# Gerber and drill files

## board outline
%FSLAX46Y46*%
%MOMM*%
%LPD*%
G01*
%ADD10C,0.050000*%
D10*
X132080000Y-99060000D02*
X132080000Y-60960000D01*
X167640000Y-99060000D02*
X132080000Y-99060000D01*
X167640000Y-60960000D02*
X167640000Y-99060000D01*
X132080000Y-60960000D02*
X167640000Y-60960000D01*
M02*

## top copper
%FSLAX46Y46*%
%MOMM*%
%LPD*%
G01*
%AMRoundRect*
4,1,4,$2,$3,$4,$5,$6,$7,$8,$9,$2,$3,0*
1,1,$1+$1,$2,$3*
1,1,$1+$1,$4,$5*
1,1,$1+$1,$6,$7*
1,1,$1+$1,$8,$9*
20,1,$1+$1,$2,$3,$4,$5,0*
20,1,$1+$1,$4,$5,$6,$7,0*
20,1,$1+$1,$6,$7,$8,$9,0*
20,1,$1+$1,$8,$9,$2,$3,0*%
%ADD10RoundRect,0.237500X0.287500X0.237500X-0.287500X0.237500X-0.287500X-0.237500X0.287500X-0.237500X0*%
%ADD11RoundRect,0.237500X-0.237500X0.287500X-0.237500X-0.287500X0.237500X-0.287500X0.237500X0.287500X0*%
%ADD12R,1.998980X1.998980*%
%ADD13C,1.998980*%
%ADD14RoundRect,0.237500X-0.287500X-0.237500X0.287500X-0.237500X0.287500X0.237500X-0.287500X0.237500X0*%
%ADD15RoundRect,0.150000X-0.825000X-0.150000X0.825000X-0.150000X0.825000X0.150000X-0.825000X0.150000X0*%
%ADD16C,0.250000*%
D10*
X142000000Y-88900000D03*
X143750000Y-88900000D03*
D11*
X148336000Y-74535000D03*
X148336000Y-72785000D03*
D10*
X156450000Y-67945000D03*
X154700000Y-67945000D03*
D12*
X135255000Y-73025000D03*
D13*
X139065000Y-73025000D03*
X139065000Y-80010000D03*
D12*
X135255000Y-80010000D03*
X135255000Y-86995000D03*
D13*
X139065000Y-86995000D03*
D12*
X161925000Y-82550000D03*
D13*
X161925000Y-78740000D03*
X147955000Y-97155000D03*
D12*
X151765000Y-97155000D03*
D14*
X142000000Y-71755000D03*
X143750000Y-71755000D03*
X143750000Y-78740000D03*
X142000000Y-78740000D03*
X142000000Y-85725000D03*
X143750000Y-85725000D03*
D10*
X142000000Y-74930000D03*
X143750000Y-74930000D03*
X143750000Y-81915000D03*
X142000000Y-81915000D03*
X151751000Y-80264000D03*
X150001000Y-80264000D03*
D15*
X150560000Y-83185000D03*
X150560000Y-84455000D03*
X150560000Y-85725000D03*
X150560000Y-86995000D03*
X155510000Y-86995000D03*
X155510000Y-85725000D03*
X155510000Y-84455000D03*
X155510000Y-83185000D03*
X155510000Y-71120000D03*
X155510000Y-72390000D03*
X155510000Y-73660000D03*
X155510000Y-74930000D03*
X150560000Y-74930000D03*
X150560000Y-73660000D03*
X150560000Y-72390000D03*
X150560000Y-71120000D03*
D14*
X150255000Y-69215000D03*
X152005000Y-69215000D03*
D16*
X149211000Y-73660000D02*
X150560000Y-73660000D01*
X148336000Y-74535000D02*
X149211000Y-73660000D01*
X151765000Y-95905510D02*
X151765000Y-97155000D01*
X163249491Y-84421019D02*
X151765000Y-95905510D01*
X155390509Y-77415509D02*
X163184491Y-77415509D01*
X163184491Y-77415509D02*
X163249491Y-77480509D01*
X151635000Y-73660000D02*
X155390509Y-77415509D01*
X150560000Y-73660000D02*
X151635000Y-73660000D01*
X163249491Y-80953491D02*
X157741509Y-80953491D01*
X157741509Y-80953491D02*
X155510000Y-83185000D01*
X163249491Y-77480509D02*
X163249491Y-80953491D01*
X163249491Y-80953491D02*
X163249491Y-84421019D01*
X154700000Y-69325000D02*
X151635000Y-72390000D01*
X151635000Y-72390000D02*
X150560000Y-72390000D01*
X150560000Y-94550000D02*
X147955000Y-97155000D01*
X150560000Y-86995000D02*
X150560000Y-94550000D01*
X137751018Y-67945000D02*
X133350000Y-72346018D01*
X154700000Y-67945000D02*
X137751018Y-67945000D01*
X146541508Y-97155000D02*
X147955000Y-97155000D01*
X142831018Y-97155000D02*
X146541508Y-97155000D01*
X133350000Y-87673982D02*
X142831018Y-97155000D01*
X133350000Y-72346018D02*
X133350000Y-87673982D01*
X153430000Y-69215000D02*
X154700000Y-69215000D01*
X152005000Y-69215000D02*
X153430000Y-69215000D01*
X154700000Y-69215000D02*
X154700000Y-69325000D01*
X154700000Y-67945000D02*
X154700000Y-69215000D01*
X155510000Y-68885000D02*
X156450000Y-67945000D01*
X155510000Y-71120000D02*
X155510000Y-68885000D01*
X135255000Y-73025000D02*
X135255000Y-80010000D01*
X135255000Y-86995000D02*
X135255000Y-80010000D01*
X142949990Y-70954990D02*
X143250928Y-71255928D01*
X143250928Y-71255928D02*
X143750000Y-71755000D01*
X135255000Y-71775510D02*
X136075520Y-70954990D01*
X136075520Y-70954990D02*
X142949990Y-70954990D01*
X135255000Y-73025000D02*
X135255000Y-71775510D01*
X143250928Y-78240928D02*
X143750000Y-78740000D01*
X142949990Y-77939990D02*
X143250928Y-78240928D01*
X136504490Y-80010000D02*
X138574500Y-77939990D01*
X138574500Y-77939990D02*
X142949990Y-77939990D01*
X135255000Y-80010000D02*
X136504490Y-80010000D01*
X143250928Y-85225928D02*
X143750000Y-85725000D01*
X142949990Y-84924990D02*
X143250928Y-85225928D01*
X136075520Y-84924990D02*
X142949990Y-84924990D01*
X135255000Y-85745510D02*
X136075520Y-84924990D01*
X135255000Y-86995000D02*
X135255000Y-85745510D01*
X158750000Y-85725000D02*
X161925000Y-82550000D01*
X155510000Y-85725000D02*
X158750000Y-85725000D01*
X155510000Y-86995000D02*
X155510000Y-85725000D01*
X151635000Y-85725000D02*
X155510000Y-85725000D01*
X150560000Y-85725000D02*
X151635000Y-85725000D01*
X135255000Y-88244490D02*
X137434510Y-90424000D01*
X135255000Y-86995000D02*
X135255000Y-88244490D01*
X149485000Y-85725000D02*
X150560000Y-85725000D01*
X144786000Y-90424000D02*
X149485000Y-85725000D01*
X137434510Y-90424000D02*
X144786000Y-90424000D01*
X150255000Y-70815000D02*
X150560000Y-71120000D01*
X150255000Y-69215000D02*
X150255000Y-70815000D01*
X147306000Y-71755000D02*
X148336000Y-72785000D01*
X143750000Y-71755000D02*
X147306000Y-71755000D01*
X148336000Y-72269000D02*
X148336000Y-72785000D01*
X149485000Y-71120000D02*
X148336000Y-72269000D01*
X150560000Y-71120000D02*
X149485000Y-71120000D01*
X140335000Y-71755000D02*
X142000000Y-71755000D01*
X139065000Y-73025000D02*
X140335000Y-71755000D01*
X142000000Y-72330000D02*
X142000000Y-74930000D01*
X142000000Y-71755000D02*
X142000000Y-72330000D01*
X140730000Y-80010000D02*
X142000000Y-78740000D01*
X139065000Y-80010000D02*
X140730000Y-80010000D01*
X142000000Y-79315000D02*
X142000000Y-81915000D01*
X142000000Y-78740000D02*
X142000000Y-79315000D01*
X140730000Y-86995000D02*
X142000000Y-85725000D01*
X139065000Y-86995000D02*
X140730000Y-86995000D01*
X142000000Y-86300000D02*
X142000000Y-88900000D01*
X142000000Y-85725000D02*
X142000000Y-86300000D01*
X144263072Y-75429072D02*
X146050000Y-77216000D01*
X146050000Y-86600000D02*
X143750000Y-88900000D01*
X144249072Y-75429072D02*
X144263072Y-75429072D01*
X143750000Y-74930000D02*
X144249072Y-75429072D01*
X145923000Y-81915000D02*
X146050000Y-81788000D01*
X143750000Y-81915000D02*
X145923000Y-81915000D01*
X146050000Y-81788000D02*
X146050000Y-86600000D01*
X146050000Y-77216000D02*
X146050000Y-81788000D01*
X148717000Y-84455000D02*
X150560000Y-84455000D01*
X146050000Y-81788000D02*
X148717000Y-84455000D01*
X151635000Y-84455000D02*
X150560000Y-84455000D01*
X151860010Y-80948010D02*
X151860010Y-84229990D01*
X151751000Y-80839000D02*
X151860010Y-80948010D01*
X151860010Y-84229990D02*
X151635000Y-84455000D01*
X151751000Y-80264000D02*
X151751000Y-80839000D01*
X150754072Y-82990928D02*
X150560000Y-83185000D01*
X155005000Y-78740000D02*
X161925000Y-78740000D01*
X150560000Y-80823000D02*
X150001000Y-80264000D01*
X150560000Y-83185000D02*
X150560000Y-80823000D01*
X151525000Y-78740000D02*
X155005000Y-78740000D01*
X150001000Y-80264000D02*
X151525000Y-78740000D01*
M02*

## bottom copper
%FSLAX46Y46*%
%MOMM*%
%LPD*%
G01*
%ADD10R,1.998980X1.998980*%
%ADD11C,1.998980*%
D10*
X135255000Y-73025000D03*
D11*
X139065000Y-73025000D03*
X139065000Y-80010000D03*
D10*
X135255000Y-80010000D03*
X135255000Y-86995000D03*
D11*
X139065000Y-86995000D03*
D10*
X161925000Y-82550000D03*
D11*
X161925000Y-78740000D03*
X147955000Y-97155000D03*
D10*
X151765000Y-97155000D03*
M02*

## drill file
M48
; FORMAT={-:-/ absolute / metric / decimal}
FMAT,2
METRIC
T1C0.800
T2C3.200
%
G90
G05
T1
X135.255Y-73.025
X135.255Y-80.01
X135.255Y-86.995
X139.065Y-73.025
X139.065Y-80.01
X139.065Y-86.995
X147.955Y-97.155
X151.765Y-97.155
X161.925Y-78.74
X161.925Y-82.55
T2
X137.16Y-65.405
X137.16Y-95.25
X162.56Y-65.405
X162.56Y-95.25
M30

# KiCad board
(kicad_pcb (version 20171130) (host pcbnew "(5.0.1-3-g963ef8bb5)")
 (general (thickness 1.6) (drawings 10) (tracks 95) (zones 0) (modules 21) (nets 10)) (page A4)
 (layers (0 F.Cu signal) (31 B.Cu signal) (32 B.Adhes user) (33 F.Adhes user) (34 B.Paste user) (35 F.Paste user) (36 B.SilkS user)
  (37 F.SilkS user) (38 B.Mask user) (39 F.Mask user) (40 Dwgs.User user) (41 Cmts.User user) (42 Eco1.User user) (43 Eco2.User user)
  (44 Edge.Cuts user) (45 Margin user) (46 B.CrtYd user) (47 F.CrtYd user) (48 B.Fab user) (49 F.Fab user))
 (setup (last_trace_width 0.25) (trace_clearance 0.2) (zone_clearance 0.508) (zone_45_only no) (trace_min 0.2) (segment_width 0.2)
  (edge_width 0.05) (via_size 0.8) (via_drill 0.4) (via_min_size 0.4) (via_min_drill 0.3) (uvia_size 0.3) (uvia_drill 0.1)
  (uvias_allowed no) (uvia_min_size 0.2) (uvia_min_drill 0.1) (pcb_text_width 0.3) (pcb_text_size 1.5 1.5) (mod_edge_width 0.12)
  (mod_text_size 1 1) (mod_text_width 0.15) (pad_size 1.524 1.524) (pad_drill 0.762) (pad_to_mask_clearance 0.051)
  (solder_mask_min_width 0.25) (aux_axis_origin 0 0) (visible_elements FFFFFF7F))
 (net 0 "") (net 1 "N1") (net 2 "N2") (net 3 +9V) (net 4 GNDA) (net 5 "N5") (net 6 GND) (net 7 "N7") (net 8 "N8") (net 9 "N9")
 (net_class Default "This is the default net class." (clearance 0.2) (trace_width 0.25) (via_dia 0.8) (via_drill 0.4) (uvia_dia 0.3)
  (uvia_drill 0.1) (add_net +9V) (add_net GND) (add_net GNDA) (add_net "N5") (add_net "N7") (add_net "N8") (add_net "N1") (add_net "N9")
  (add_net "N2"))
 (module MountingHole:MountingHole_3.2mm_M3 (layer F.Cu) (at 162.56 95.25)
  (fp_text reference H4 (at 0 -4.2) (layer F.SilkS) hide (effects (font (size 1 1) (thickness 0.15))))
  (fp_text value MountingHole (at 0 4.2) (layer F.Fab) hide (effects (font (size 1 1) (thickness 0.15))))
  (pad 1 np_thru_hole circle (at 0 0) (size 3.2 3.2) (drill 3.2) (layers *.Cu *.Mask)))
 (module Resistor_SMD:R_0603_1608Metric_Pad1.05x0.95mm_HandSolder (layer F.Cu) (at 142.875 88.9 180)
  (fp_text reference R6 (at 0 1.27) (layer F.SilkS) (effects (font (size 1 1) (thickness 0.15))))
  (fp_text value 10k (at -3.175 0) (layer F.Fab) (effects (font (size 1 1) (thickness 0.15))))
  (pad 2 smd roundrect (at 0.875 0 180) (size 1.05 0.95) (layers F.Cu F.Paste F.Mask) (roundrect_rratio 0.25) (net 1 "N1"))
  (pad 1 smd roundrect (at -0.875 0 180) (size 1.05 0.95) (layers F.Cu F.Paste F.Mask) (roundrect_rratio 0.25) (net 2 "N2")))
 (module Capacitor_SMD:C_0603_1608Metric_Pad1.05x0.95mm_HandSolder (layer F.Cu) (at 148.336 73.66 270)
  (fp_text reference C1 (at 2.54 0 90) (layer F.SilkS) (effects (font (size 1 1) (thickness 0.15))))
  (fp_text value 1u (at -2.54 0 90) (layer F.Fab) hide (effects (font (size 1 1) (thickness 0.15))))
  (pad 2 smd roundrect (at 0.875 0 270) (size 1.05 0.95) (layers F.Cu F.Paste F.Mask) (roundrect_rratio 0.25) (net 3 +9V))
  (pad 1 smd roundrect (at -0.875 0 270) (size 1.05 0.95) (layers F.Cu F.Paste F.Mask) (roundrect_rratio 0.25) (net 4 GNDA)))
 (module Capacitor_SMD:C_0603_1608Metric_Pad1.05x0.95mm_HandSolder (layer F.Cu) (at 155.575 67.945 180)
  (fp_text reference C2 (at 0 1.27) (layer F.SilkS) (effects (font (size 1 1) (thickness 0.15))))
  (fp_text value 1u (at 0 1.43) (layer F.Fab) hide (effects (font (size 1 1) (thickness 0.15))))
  (pad 1 smd roundrect (at -0.875 0 180) (size 1.05 0.95) (layers F.Cu F.Paste F.Mask) (roundrect_rratio 0.25) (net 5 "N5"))
  (pad 2 smd roundrect (at 0.875 0 180) (size 1.05 0.95) (layers F.Cu F.Paste F.Mask) (roundrect_rratio 0.25) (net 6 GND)))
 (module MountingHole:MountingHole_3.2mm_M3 (layer F.Cu) (at 137.16 65.405)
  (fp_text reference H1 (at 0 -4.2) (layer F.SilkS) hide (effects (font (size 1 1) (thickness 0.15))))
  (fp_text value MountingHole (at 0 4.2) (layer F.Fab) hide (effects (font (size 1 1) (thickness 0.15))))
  (pad 1 np_thru_hole circle (at 0 0) (size 3.2 3.2) (drill 3.2) (layers *.Cu *.Mask)))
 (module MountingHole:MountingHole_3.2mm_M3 (layer F.Cu) (at 162.56 65.405)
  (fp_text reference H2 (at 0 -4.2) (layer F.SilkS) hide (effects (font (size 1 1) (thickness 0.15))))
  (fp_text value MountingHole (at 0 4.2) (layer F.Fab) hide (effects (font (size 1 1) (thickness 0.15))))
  (pad 1 np_thru_hole circle (at 0 0) (size 3.2 3.2) (drill 3.2) (layers *.Cu *.Mask)))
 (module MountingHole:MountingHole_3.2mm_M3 (layer F.Cu) (at 137.16 95.25)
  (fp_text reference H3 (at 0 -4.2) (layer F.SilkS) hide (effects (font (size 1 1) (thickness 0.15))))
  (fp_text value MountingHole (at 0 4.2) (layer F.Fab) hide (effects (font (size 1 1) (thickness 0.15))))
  (pad 1 np_thru_hole circle (at 0 0) (size 3.2 3.2) (drill 3.2) (layers *.Cu *.Mask)))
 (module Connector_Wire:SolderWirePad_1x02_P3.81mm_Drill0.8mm (layer F.Cu) (at 135.255 73.025)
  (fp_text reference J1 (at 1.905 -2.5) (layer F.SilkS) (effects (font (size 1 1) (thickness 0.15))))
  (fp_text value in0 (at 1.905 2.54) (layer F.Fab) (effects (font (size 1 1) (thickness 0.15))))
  (pad 1 thru_hole rect (at 0 0) (size 1.99898 1.99898) (drill 0.8001) (layers *.Cu *.Mask) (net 4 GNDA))
  (pad 2 thru_hole circle (at 3.81 0) (size 1.99898 1.99898) (drill 0.8001) (layers *.Cu *.Mask) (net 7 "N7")))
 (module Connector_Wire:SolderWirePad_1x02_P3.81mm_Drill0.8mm (layer F.Cu) (at 135.255 80.01)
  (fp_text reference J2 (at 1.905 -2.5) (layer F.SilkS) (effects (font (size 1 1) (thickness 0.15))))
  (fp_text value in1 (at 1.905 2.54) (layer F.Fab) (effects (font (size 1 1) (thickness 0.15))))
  (pad 2 thru_hole circle (at 3.81 0) (size 1.99898 1.99898) (drill 0.8001) (layers *.Cu *.Mask) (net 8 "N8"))
  (pad 1 thru_hole rect (at 0 0) (size 1.99898 1.99898) (drill 0.8001) (layers *.Cu *.Mask) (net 4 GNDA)))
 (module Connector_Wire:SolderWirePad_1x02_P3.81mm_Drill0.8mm (layer F.Cu) (at 135.255 86.995)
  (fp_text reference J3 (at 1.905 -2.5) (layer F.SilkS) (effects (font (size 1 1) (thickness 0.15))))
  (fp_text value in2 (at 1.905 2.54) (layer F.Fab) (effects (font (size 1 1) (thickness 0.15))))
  (pad 1 thru_hole rect (at 0 0) (size 1.99898 1.99898) (drill 0.8001) (layers *.Cu *.Mask) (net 4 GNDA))
  (pad 2 thru_hole circle (at 3.81 0) (size 1.99898 1.99898) (drill 0.8001) (layers *.Cu *.Mask) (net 1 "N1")))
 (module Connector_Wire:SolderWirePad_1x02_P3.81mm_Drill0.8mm (layer F.Cu) (at 161.925 82.55 90)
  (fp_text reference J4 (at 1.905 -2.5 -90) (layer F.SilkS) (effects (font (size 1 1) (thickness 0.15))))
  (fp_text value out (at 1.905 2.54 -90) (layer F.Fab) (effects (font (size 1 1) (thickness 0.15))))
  (pad 1 thru_hole rect (at 0 0 90) (size 1.99898 1.99898) (drill 0.8001) (layers *.Cu *.Mask) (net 4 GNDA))
  (pad 2 thru_hole circle (at 3.81 0 90) (size 1.99898 1.99898) (drill 0.8001) (layers *.Cu *.Mask) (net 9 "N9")))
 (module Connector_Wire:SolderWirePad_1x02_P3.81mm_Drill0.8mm (layer F.Cu) (at 151.765 97.155 180)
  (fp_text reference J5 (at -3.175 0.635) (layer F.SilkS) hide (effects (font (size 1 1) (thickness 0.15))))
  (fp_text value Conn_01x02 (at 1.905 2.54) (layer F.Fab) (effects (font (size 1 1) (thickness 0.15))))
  (pad 2 thru_hole circle (at 3.81 0 180) (size 1.99898 1.99898) (drill 0.8001) (layers *.Cu *.Mask) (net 6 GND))
  (pad 1 thru_hole rect (at 0 0 180) (size 1.99898 1.99898) (drill 0.8001) (layers *.Cu *.Mask) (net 3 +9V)))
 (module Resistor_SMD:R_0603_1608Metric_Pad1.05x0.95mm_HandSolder (layer F.Cu) (at 142.875 71.755)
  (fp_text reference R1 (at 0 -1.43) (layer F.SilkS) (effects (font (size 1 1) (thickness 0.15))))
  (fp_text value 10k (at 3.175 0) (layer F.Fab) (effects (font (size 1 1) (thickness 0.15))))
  (pad 1 smd roundrect (at -0.875 0) (size 1.05 0.95) (layers F.Cu F.Paste F.Mask) (roundrect_rratio 0.25) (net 7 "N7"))
  (pad 2 smd roundrect (at 0.875 0) (size 1.05 0.95) (layers F.Cu F.Paste F.Mask) (roundrect_rratio 0.25) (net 4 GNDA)))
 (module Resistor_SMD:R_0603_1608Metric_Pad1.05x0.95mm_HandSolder (layer F.Cu) (at 142.875 78.74)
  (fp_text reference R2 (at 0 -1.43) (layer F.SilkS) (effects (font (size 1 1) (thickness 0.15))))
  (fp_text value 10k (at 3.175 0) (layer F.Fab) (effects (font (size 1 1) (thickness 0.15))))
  (pad 2 smd roundrect (at 0.875 0) (size 1.05 0.95) (layers F.Cu F.Paste F.Mask) (roundrect_rratio 0.25) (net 4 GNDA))
  (pad 1 smd roundrect (at -0.875 0) (size 1.05 0.95) (layers F.Cu F.Paste F.Mask) (roundrect_rratio 0.25) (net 8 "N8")))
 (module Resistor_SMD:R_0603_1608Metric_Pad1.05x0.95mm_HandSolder (layer F.Cu) (at 142.875 85.725)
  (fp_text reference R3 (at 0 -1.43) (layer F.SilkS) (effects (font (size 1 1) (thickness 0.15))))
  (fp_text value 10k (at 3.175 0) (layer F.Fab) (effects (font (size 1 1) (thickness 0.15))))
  (pad 1 smd roundrect (at -0.875 0) (size 1.05 0.95) (layers F.Cu F.Paste F.Mask) (roundrect_rratio 0.25) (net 1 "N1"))
  (pad 2 smd roundrect (at 0.875 0) (size 1.05 0.95) (layers F.Cu F.Paste F.Mask) (roundrect_rratio 0.25) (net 4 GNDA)))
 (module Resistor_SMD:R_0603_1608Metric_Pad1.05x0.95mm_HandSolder (layer F.Cu) (at 142.875 74.93 180)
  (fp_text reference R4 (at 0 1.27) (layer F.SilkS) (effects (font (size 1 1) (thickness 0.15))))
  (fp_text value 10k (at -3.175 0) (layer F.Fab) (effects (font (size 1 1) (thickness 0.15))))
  (pad 2 smd roundrect (at 0.875 0 180) (size 1.05 0.95) (layers F.Cu F.Paste F.Mask) (roundrect_rratio 0.25) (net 7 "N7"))
  (pad 1 smd roundrect (at -0.875 0 180) (size 1.05 0.95) (layers F.Cu F.Paste F.Mask) (roundrect_rratio 0.25) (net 2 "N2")))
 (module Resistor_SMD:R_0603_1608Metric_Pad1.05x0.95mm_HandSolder (layer F.Cu) (at 142.875 81.915 180)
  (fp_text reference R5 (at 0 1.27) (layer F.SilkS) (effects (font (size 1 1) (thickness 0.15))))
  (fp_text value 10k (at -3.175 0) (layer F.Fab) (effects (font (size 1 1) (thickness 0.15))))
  (pad 1 smd roundrect (at -0.875 0 180) (size 1.05 0.95) (layers F.Cu F.Paste F.Mask) (roundrect_rratio 0.25) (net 2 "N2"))
  (pad 2 smd roundrect (at 0.875 0 180) (size 1.05 0.95) (layers F.Cu F.Paste F.Mask) (roundrect_rratio 0.25) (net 8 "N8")))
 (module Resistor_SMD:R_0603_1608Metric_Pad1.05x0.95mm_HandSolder (layer F.Cu) (at 150.876 80.264 180)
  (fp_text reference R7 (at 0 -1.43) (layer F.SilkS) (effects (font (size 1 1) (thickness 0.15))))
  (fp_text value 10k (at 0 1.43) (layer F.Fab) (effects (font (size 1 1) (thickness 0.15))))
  (pad 1 smd roundrect (at -0.875 0 180) (size 1.05 0.95) (layers F.Cu F.Paste F.Mask) (roundrect_rratio 0.25) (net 2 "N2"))
  (pad 2 smd roundrect (at 0.875 0 180) (size 1.05 0.95) (layers F.Cu F.Paste F.Mask) (roundrect_rratio 0.25) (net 9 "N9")))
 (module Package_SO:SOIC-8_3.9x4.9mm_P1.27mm (layer F.Cu) (at 153.035 85.09)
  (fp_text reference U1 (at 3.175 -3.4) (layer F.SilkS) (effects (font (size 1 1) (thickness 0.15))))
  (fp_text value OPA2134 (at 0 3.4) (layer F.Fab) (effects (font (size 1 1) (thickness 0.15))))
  (pad 1 smd roundrect (at -2.475 -1.905) (size 1.95 0.6) (layers F.Cu F.Paste F.Mask) (roundrect_rratio 0.25) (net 9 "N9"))
  (pad 2 smd roundrect (at -2.475 -0.635) (size 1.95 0.6) (layers F.Cu F.Paste F.Mask) (roundrect_rratio 0.25) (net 2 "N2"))
  (pad 3 smd roundrect (at -2.475 0.635) (size 1.95 0.6) (layers F.Cu F.Paste F.Mask) (roundrect_rratio 0.25) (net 4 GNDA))
  (pad 4 smd roundrect (at -2.475 1.905) (size 1.95 0.6) (layers F.Cu F.Paste F.Mask) (roundrect_rratio 0.25) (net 6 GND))
  (pad 5 smd roundrect (at 2.475 1.905) (size 1.95 0.6) (layers F.Cu F.Paste F.Mask) (roundrect_rratio 0.25) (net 4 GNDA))
  (pad 6 smd roundrect (at 2.475 0.635) (size 1.95 0.6) (layers F.Cu F.Paste F.Mask) (roundrect_rratio 0.25) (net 4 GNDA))
  (pad 7 smd roundrect (at 2.475 -0.635) (size 1.95 0.6) (layers F.Cu F.Paste F.Mask) (roundrect_rratio 0.25))
  (pad 8 smd roundrect (at 2.475 -1.905) (size 1.95 0.6) (layers F.Cu F.Paste F.Mask) (roundrect_rratio 0.25) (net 3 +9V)))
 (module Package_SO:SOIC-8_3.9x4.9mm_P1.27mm (layer F.Cu) (at 153.035 73.025)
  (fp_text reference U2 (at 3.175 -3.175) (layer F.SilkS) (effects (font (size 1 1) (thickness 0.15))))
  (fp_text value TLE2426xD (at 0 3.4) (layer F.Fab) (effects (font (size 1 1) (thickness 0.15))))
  (pad 8 smd roundrect (at 2.475 -1.905) (size 1.95 0.6) (layers F.Cu F.Paste F.Mask) (roundrect_rratio 0.25) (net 5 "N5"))
  (pad 7 smd roundrect (at 2.475 -0.635) (size 1.95 0.6) (layers F.Cu F.Paste F.Mask) (roundrect_rratio 0.25))
  (pad 6 smd roundrect (at 2.475 0.635) (size 1.95 0.6) (layers F.Cu F.Paste F.Mask) (roundrect_rratio 0.25))
  (pad 5 smd roundrect (at 2.475 1.905) (size 1.95 0.6) (layers F.Cu F.Paste F.Mask) (roundrect_rratio 0.25))
  (pad 4 smd roundrect (at -2.475 1.905) (size 1.95 0.6) (layers F.Cu F.Paste F.Mask) (roundrect_rratio 0.25))
  (pad 3 smd roundrect (at -2.475 0.635) (size 1.95 0.6) (layers F.Cu F.Paste F.Mask) (roundrect_rratio 0.25) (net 3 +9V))
  (pad 2 smd roundrect (at -2.475 -0.635) (size 1.95 0.6) (layers F.Cu F.Paste F.Mask) (roundrect_rratio 0.25) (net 6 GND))
  (pad 1 smd roundrect (at -2.475 -1.905) (size 1.95 0.6) (layers F.Cu F.Paste F.Mask) (roundrect_rratio 0.25) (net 4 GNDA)))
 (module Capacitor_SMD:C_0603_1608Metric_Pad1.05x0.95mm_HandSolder (layer F.Cu) (at 151.13 69.215)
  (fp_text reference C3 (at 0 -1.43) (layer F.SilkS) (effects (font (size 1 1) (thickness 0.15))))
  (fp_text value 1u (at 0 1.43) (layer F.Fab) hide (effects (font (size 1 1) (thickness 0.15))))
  (pad 1 smd roundrect (at -0.875 0) (size 1.05 0.95) (layers F.Cu F.Paste F.Mask) (roundrect_rratio 0.25) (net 4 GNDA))
  (pad 2 smd roundrect (at 0.875 0) (size 1.05 0.95) (layers F.Cu F.Paste F.Mask) (roundrect_rratio 0.25) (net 6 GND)))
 (gr_line (start 132.08 99.06) (end 132.08 60.96) (layer Edge.Cuts) (width 0.05))
 (gr_line (start 167.64 99.06) (end 132.08 99.06) (layer Edge.Cuts) (width 0.05))
 (gr_line (start 167.64 60.96) (end 167.64 99.06) (layer Edge.Cuts) (width 0.05))
 (gr_line (start 132.08 60.96) (end 167.64 60.96) (layer Edge.Cuts) (width 0.05))
 (segment (start 149.211 73.66) (end 150.56 73.66) (width 0.25) (layer F.Cu) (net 3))
 (segment (start 148.336 74.535) (end 149.211 73.66) (width 0.25) (layer F.Cu) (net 3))
 (segment (start 151.765 95.90551) (end 151.765 97.155) (width 0.25) (layer F.Cu) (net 3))
 (segment (start 163.249491 84.421019) (end 151.765 95.90551) (width 0.25) (layer F.Cu) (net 3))
 (segment (start 155.390509 77.415509) (end 163.184491 77.415509) (width 0.25) (layer F.Cu) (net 3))
 (segment (start 163.184491 77.415509) (end 163.249491 77.480509) (width 0.25) (layer F.Cu) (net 3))
 (segment (start 151.635 73.66) (end 155.390509 77.415509) (width 0.25) (layer F.Cu) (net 3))
 (segment (start 150.56 73.66) (end 151.635 73.66) (width 0.25) (layer F.Cu) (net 3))
 (segment (start 163.249491 80.953491) (end 157.741509 80.953491) (width 0.25) (layer F.Cu) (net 3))
 (segment (start 157.741509 80.953491) (end 155.51 83.185) (width 0.25) (layer F.Cu) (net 3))
 (segment (start 163.249491 77.480509) (end 163.249491 80.953491) (width 0.25) (layer F.Cu) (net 3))
 (segment (start 163.249491 80.953491) (end 163.249491 84.421019) (width 0.25) (layer F.Cu) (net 3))
 (segment (start 154.7 69.325) (end 151.635 72.39) (width 0.25) (layer F.Cu) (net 6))
 (segment (start 151.635 72.39) (end 150.56 72.39) (width 0.25) (layer F.Cu) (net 6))
 (segment (start 150.56 94.55) (end 147.955 97.155) (width 0.25) (layer F.Cu) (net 6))
 (segment (start 150.56 86.995) (end 150.56 94.55) (width 0.25) (layer F.Cu) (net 6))
 (segment (start 137.751018 67.945) (end 133.35 72.346018) (width 0.25) (layer F.Cu) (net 6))
 (segment (start 154.7 67.945) (end 137.751018 67.945) (width 0.25) (layer F.Cu) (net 6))
 (segment (start 146.541508 97.155) (end 147.955 97.155) (width 0.25) (layer F.Cu) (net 6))
 (segment (start 142.831018 97.155) (end 146.541508 97.155) (width 0.25) (layer F.Cu) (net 6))
 (segment (start 133.35 87.673982) (end 142.831018 97.155) (width 0.25) (layer F.Cu) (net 6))
 (segment (start 133.35 72.346018) (end 133.35 87.673982) (width 0.25) (layer F.Cu) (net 6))
 (segment (start 153.43 69.215) (end 154.7 69.215) (width 0.25) (layer F.Cu) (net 6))
 (segment (start 152.005 69.215) (end 153.43 69.215) (width 0.25) (layer F.Cu) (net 6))
 (segment (start 154.7 69.215) (end 154.7 69.325) (width 0.25) (layer F.Cu) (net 6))
 (segment (start 154.7 67.945) (end 154.7 69.215) (width 0.25) (layer F.Cu) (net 6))
 (segment (start 155.51 68.885) (end 156.45 67.945) (width 0.25) (layer F.Cu) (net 5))
 (segment (start 155.51 71.12) (end 155.51 68.885) (width 0.25) (layer F.Cu) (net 5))
 (segment (start 135.255 73.025) (end 135.255 80.01) (width 0.25) (layer F.Cu) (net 4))
 (segment (start 135.255 86.995) (end 135.255 80.01) (width 0.25) (layer F.Cu) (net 4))
 (segment (start 142.94999 70.95499) (end 143.250928 71.255928) (width 0.25) (layer F.Cu) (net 4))
 (segment (start 143.250928 71.255928) (end 143.75 71.755) (width 0.25) (layer F.Cu) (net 4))
 (segment (start 135.255 71.77551) (end 136.07552 70.95499) (width 0.25) (layer F.Cu) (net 4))
 (segment (start 136.07552 70.95499) (end 142.94999 70.95499) (width 0.25) (layer F.Cu) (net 4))
 (segment (start 135.255 73.025) (end 135.255 71.77551) (width 0.25) (layer F.Cu) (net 4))
 (segment (start 143.250928 78.240928) (end 143.75 78.74) (width 0.25) (layer F.Cu) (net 4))
 (segment (start 142.94999 77.93999) (end 143.250928 78.240928) (width 0.25) (layer F.Cu) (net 4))
 (segment (start 136.50449 80.01) (end 138.5745 77.93999) (width 0.25) (layer F.Cu) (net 4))
 (segment (start 138.5745 77.93999) (end 142.94999 77.93999) (width 0.25) (layer F.Cu) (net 4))
 (segment (start 135.255 80.01) (end 136.50449 80.01) (width 0.25) (layer F.Cu) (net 4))
 (segment (start 143.250928 85.225928) (end 143.75 85.725) (width 0.25) (layer F.Cu) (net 4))
 (segment (start 142.94999 84.92499) (end 143.250928 85.225928) (width 0.25) (layer F.Cu) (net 4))
 (segment (start 136.07552 84.92499) (end 142.94999 84.92499) (width 0.25) (layer F.Cu) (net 4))
 (segment (start 135.255 85.74551) (end 136.07552 84.92499) (width 0.25) (layer F.Cu) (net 4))
 (segment (start 135.255 86.995) (end 135.255 85.74551) (width 0.25) (layer F.Cu) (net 4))
 (segment (start 158.75 85.725) (end 161.925 82.55) (width 0.25) (layer F.Cu) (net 4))
 (segment (start 155.51 85.725) (end 158.75 85.725) (width 0.25) (layer F.Cu) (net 4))
 (segment (start 155.51 86.995) (end 155.51 85.725) (width 0.25) (layer F.Cu) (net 4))
 (segment (start 151.635 85.725) (end 155.51 85.725) (width 0.25) (layer F.Cu) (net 4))
 (segment (start 150.56 85.725) (end 151.635 85.725) (width 0.25) (layer F.Cu) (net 4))
 (segment (start 135.255 88.24449) (end 137.43451 90.424) (width 0.25) (layer F.Cu) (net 4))
 (segment (start 135.255 86.995) (end 135.255 88.24449) (width 0.25) (layer F.Cu) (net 4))
 (segment (start 149.485 85.725) (end 150.56 85.725) (width 0.25) (layer F.Cu) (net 4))
 (segment (start 144.786 90.424) (end 149.485 85.725) (width 0.25) (layer F.Cu) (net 4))
 (segment (start 137.43451 90.424) (end 144.786 90.424) (width 0.25) (layer F.Cu) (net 4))
 (segment (start 150.255 70.815) (end 150.56 71.12) (width 0.25) (layer F.Cu) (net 4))
 (segment (start 150.255 69.215) (end 150.255 70.815) (width 0.25) (layer F.Cu) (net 4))
 (segment (start 147.306 71.755) (end 148.336 72.785) (width 0.25) (layer F.Cu) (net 4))
 (segment (start 143.75 71.755) (end 147.306 71.755) (width 0.25) (layer F.Cu) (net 4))
 (segment (start 148.336 72.269) (end 148.336 72.785) (width 0.25) (layer F.Cu) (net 4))
 (segment (start 149.485 71.12) (end 148.336 72.269) (width 0.25) (layer F.Cu) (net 4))
 (segment (start 150.56 71.12) (end 149.485 71.12) (width 0.25) (layer F.Cu) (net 4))
 (segment (start 140.335 71.755) (end 142 71.755) (width 0.25) (layer F.Cu) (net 7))
 (segment (start 139.065 73.025) (end 140.335 71.755) (width 0.25) (layer F.Cu) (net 7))
 (segment (start 142 72.33) (end 142 74.93) (width 0.25) (layer F.Cu) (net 7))
 (segment (start 142 71.755) (end 142 72.33) (width 0.25) (layer F.Cu) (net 7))
 (segment (start 140.73 80.01) (end 142 78.74) (width 0.25) (layer F.Cu) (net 8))
 (segment (start 139.065 80.01) (end 140.73 80.01) (width 0.25) (layer F.Cu) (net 8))
 (segment (start 142 79.315) (end 142 81.915) (width 0.25) (layer F.Cu) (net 8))
 (segment (start 142 78.74) (end 142 79.315) (width 0.25) (layer F.Cu) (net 8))
 (segment (start 140.73 86.995) (end 142 85.725) (width 0.25) (layer F.Cu) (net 1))
 (segment (start 139.065 86.995) (end 140.73 86.995) (width 0.25) (layer F.Cu) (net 1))
 (segment (start 142 86.3) (end 142 88.9) (width 0.25) (layer F.Cu) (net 1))
 (segment (start 142 85.725) (end 142 86.3) (width 0.25) (layer F.Cu) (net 1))
 (segment (start 144.263072 75.429072) (end 146.05 77.216) (width 0.25) (layer F.Cu) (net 2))
 (segment (start 146.05 86.6) (end 143.75 88.9) (width 0.25) (layer F.Cu) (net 2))
 (segment (start 144.249072 75.429072) (end 144.263072 75.429072) (width 0.25) (layer F.Cu) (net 2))
 (segment (start 143.75 74.93) (end 144.249072 75.429072) (width 0.25) (layer F.Cu) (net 2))
 (segment (start 145.923 81.915) (end 146.05 81.788) (width 0.25) (layer F.Cu) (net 2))
 (segment (start 143.75 81.915) (end 145.923 81.915) (width 0.25) (layer F.Cu) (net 2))
 (segment (start 146.05 81.788) (end 146.05 86.6) (width 0.25) (layer F.Cu) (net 2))
 (segment (start 146.05 77.216) (end 146.05 81.788) (width 0.25) (layer F.Cu) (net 2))
 (segment (start 148.717 84.455) (end 150.56 84.455) (width 0.25) (layer F.Cu) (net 2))
 (segment (start 146.05 81.788) (end 148.717 84.455) (width 0.25) (layer F.Cu) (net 2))
 (segment (start 151.635 84.455) (end 150.56 84.455) (width 0.25) (layer F.Cu) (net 2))
 (segment (start 151.86001 80.94801) (end 151.86001 84.22999) (width 0.25) (layer F.Cu) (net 2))
 (segment (start 151.751 80.839) (end 151.86001 80.94801) (width 0.25) (layer F.Cu) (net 2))
 (segment (start 151.86001 84.22999) (end 151.635 84.455) (width 0.25) (layer F.Cu) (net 2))
 (segment (start 151.751 80.264) (end 151.751 80.839) (width 0.25) (layer F.Cu) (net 2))
 (segment (start 150.754072 82.990928) (end 150.56 83.185) (width 0.25) (layer F.Cu) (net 9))
 (segment (start 155.005 78.74) (end 161.925 78.74) (width 0.25) (layer F.Cu) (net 9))
 (segment (start 150.56 80.823) (end 150.001 80.264) (width 0.25) (layer F.Cu) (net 9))
 (segment (start 150.56 83.185) (end 150.56 80.823) (width 0.25) (layer F.Cu) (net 9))
 (segment (start 151.525 78.74) (end 155.005 78.74) (width 0.25) (layer F.Cu) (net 9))
 (segment (start 150.001 80.264) (end 151.525 78.74) (width 0.25) (layer F.Cu) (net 9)))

